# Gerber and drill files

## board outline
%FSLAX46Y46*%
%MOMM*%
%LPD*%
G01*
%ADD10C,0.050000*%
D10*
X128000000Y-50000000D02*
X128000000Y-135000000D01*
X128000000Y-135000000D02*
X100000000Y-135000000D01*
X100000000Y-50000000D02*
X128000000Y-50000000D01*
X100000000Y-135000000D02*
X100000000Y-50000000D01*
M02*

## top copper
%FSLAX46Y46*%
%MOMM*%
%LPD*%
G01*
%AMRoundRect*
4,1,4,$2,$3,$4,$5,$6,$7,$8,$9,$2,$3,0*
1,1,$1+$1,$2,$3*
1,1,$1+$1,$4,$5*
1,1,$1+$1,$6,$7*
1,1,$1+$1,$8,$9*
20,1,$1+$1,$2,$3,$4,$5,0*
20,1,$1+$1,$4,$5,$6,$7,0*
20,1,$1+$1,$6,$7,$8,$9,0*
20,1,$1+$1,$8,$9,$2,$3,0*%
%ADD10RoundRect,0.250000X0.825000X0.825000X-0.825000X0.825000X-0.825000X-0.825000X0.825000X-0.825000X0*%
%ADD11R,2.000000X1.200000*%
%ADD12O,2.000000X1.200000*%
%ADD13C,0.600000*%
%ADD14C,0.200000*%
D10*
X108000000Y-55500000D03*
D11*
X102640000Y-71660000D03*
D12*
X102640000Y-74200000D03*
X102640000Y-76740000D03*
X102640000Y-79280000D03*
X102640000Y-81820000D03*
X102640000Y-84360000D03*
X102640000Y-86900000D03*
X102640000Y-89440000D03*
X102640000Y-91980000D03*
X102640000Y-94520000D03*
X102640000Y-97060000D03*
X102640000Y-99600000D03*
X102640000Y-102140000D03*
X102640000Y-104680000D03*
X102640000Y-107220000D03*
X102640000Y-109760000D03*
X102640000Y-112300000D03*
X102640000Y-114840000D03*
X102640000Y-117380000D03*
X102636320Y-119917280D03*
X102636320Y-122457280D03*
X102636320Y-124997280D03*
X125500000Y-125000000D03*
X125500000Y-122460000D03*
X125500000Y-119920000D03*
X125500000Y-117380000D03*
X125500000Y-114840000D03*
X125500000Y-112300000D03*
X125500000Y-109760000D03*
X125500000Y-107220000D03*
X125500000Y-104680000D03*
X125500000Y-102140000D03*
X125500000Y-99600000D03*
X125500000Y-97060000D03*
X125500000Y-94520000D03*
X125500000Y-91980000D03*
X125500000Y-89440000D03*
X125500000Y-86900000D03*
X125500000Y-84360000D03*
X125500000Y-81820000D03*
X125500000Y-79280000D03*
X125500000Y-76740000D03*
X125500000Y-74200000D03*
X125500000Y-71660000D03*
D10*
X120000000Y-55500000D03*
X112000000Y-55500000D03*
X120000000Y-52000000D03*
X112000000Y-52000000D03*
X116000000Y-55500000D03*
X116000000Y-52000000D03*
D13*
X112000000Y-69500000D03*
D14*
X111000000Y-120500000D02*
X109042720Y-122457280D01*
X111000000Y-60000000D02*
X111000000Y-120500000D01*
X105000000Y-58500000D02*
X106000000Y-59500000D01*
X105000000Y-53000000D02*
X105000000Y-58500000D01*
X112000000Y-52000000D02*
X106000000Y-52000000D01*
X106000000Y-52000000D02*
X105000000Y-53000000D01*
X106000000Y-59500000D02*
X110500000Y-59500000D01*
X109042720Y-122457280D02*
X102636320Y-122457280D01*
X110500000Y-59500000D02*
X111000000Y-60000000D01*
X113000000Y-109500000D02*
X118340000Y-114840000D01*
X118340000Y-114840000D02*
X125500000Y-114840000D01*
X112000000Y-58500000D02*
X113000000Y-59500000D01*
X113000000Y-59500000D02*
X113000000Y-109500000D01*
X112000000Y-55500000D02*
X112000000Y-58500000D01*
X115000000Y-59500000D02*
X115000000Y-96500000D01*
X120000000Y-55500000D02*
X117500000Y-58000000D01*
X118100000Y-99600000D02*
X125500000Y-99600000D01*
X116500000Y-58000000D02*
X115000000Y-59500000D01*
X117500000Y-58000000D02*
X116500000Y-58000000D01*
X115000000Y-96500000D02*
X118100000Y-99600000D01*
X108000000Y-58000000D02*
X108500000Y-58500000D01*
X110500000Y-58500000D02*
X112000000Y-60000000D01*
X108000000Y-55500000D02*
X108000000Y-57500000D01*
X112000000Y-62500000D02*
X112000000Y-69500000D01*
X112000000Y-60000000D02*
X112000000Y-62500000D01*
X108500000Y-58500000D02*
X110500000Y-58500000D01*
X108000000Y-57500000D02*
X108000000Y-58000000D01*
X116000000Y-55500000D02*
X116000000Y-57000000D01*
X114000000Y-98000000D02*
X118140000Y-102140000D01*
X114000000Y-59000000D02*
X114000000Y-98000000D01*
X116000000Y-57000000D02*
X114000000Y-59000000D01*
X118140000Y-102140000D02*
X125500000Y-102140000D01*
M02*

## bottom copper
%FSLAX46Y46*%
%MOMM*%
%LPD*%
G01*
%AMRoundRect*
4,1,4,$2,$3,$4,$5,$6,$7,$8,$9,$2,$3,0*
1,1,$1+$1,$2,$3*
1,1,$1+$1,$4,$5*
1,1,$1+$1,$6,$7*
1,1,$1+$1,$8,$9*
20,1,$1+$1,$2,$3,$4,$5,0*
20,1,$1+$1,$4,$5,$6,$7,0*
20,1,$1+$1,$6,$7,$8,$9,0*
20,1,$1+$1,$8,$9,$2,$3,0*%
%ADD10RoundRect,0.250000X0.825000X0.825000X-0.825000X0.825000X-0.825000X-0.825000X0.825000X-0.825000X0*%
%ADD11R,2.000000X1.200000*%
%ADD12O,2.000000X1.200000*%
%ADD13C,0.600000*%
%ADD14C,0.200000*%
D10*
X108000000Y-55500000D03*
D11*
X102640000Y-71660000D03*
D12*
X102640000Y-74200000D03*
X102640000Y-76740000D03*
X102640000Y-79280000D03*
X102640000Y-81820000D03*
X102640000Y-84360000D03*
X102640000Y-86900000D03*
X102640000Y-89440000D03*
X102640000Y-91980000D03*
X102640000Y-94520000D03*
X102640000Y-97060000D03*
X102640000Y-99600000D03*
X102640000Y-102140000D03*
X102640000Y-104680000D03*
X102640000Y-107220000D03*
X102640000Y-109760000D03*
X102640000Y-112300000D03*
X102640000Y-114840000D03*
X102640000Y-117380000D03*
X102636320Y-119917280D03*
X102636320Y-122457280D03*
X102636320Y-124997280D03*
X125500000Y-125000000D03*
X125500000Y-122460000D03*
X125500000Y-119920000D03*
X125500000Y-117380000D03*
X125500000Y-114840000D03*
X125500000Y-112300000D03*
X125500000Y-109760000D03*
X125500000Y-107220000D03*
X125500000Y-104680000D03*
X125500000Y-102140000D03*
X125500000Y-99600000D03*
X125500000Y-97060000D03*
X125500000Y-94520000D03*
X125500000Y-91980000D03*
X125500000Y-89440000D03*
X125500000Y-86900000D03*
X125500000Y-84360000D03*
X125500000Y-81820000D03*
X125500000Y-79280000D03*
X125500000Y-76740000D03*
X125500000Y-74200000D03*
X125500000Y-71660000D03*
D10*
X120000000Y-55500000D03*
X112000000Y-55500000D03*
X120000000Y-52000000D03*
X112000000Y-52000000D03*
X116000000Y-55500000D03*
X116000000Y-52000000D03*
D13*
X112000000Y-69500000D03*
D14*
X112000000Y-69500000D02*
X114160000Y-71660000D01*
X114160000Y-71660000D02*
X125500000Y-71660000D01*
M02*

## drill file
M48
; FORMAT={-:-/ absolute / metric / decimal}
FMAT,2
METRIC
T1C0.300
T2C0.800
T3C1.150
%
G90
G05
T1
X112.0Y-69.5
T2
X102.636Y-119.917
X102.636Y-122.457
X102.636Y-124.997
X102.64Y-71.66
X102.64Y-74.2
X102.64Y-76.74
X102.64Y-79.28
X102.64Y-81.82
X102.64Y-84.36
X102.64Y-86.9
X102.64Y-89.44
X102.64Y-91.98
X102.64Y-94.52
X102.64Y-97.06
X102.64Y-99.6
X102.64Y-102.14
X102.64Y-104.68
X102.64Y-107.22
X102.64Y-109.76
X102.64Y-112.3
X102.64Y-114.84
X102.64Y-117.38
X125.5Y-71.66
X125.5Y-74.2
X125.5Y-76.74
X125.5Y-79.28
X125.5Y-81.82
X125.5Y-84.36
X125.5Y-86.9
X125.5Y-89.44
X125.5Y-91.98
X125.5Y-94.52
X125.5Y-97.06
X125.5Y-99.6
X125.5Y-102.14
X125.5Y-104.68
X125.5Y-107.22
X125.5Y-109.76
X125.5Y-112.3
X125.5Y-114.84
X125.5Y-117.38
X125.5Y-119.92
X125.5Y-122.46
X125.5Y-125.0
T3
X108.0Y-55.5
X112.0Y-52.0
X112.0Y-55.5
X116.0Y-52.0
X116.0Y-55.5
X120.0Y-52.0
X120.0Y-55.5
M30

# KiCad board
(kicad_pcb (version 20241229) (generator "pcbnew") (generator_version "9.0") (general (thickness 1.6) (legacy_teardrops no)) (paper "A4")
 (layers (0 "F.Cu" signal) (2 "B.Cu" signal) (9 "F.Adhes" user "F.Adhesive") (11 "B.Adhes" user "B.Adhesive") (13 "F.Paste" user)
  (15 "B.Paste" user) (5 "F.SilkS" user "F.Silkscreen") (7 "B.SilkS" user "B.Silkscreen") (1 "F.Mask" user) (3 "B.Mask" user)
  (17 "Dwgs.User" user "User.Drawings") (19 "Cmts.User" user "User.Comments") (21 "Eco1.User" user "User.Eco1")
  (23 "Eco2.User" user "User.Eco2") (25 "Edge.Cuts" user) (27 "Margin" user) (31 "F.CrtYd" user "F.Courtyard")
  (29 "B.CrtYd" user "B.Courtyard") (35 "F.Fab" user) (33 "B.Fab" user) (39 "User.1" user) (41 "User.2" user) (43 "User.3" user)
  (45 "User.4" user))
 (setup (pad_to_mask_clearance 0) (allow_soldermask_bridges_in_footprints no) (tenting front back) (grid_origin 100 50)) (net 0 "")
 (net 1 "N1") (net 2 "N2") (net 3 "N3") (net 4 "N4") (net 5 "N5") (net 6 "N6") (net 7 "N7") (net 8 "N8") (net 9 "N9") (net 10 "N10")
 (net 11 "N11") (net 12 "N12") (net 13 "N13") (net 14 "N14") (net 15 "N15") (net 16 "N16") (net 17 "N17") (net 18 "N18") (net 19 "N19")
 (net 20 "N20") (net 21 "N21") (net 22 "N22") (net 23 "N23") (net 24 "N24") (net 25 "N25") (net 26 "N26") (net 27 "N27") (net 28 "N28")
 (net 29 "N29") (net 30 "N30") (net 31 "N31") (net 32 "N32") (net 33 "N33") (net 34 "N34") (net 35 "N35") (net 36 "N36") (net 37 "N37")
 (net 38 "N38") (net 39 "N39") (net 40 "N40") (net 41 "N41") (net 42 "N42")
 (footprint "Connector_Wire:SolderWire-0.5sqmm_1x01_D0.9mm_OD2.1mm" (layer "F.Cu") (at 108 55.5 180)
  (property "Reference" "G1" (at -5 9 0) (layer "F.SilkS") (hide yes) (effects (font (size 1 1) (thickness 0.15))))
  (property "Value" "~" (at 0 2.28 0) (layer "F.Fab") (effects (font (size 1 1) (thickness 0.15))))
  (pad "1" thru_hole roundrect (at 0 0 180) (size 2.15 2.15) (drill 1.15) (layers "*.Cu" "*.Mask") (remove_unused_layers no)
   (roundrect_rratio 0.116279) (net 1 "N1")))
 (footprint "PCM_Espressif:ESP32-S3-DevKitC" (layer "F.Cu") (at 102.64 71.66)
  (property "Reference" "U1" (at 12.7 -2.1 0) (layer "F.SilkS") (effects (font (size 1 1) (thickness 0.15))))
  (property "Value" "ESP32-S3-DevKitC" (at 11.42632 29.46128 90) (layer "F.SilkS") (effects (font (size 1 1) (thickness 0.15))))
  (pad "1" thru_hole rect (at 0 0 270) (size 1.2 2) (drill 0.8) (layers "*.Cu" "*.Mask") (remove_unused_layers no) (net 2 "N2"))
  (pad "2" thru_hole oval (at 0 2.54 270) (size 1.2 2) (drill 0.8) (layers "*.Cu" "*.Mask") (remove_unused_layers no) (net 2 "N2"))
  (pad "3" thru_hole oval (at 0 5.08 270) (size 1.2 2) (drill 0.8) (layers "*.Cu" "*.Mask") (remove_unused_layers no) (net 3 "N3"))
  (pad "4" thru_hole oval (at 0 7.62 270) (size 1.2 2) (drill 0.8) (layers "*.Cu" "*.Mask") (remove_unused_layers no) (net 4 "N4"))
  (pad "5" thru_hole oval (at 0 10.16 270) (size 1.2 2) (drill 0.8) (layers "*.Cu" "*.Mask") (remove_unused_layers no) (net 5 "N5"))
  (pad "6" thru_hole oval (at 0 12.7 270) (size 1.2 2) (drill 0.8) (layers "*.Cu" "*.Mask") (remove_unused_layers no) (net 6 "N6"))
  (pad "7" thru_hole oval (at 0 15.24 270) (size 1.2 2) (drill 0.8) (layers "*.Cu" "*.Mask") (remove_unused_layers no) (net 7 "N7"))
  (pad "8" thru_hole oval (at 0 17.78 270) (size 1.2 2) (drill 0.8) (layers "*.Cu" "*.Mask") (remove_unused_layers no) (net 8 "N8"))
  (pad "9" thru_hole oval (at 0 20.32 270) (size 1.2 2) (drill 0.8) (layers "*.Cu" "*.Mask") (remove_unused_layers no) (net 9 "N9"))
  (pad "10" thru_hole oval (at 0 22.86 270) (size 1.2 2) (drill 0.8) (layers "*.Cu" "*.Mask") (remove_unused_layers no) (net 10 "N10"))
  (pad "11" thru_hole oval (at 0 25.4 270) (size 1.2 2) (drill 0.8) (layers "*.Cu" "*.Mask") (remove_unused_layers no) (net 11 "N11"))
  (pad "12" thru_hole oval (at 0 27.94 270) (size 1.2 2) (drill 0.8) (layers "*.Cu" "*.Mask") (remove_unused_layers no) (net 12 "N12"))
  (pad "13" thru_hole oval (at 0 30.48 270) (size 1.2 2) (drill 0.8) (layers "*.Cu" "*.Mask") (remove_unused_layers no) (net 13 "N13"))
  (pad "14" thru_hole oval (at 0 33.02 270) (size 1.2 2) (drill 0.8) (layers "*.Cu" "*.Mask") (remove_unused_layers no) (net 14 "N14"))
  (pad "15" thru_hole oval (at 0 35.56 270) (size 1.2 2) (drill 0.8) (layers "*.Cu" "*.Mask") (remove_unused_layers no) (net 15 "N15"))
  (pad "16" thru_hole oval (at 0 38.1 270) (size 1.2 2) (drill 0.8) (layers "*.Cu" "*.Mask") (remove_unused_layers no) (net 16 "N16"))
  (pad "17" thru_hole oval (at 0 40.64 270) (size 1.2 2) (drill 0.8) (layers "*.Cu" "*.Mask") (remove_unused_layers no) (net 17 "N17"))
  (pad "18" thru_hole oval (at 0 43.18 270) (size 1.2 2) (drill 0.8) (layers "*.Cu" "*.Mask") (remove_unused_layers no) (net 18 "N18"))
  (pad "19" thru_hole oval (at 0 45.72 270) (size 1.2 2) (drill 0.8) (layers "*.Cu" "*.Mask") (remove_unused_layers no) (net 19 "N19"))
  (pad "20" thru_hole oval (at -0.00368 48.25728 270) (size 1.2 2) (drill 0.8) (layers "*.Cu" "*.Mask") (remove_unused_layers no)
   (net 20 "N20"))
  (pad "21" thru_hole oval (at -0.00368 50.79728 270) (size 1.2 2) (drill 0.8) (layers "*.Cu" "*.Mask") (remove_unused_layers no)
   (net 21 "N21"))
  (pad "22" thru_hole oval (at -0.00368 53.33728 270) (size 1.2 2) (drill 0.8) (layers "*.Cu" "*.Mask") (remove_unused_layers no)
   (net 1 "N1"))
  (pad "23" thru_hole oval (at 22.86 53.34 270) (size 1.2 2) (drill 0.8) (layers "*.Cu" "*.Mask") (remove_unused_layers no) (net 1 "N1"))
  (pad "24" thru_hole oval (at 22.86 50.8 270) (size 1.2 2) (drill 0.8) (layers "*.Cu" "*.Mask") (remove_unused_layers no) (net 1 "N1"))
  (pad "25" thru_hole oval (at 22.86 48.26 270) (size 1.2 2) (drill 0.8) (layers "*.Cu" "*.Mask") (remove_unused_layers no) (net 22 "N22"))
  (pad "26" thru_hole oval (at 22.86 45.72 270) (size 1.2 2) (drill 0.8) (layers "*.Cu" "*.Mask") (remove_unused_layers no) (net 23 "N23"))
  (pad "27" thru_hole oval (at 22.86 43.18 270) (size 1.2 2) (drill 0.8) (layers "*.Cu" "*.Mask") (remove_unused_layers no) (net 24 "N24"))
  (pad "28" thru_hole oval (at 22.86 40.64 270) (size 1.2 2) (drill 0.8) (layers "*.Cu" "*.Mask") (remove_unused_layers no) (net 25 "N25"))
  (pad "29" thru_hole oval (at 22.86 38.1 270) (size 1.2 2) (drill 0.8) (layers "*.Cu" "*.Mask") (remove_unused_layers no) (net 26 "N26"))
  (pad "30" thru_hole oval (at 22.86 35.56 270) (size 1.2 2) (drill 0.8) (layers "*.Cu" "*.Mask") (remove_unused_layers no) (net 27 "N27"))
  (pad "31" thru_hole oval (at 22.86 33.02 270) (size 1.2 2) (drill 0.8) (layers "*.Cu" "*.Mask") (remove_unused_layers no) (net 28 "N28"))
  (pad "32" thru_hole oval (at 22.86 30.48 270) (size 1.2 2) (drill 0.8) (layers "*.Cu" "*.Mask") (remove_unused_layers no) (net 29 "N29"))
  (pad "33" thru_hole oval (at 22.86 27.94 270) (size 1.2 2) (drill 0.8) (layers "*.Cu" "*.Mask") (remove_unused_layers no) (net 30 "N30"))
  (pad "34" thru_hole oval (at 22.86 25.4 270) (size 1.2 2) (drill 0.8) (layers "*.Cu" "*.Mask") (remove_unused_layers no) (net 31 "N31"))
  (pad "35" thru_hole oval (at 22.86 22.86 270) (size 1.2 2) (drill 0.8) (layers "*.Cu" "*.Mask") (remove_unused_layers no) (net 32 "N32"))
  (pad "36" thru_hole oval (at 22.86 20.32 270) (size 1.2 2) (drill 0.8) (layers "*.Cu" "*.Mask") (remove_unused_layers no) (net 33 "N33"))
  (pad "37" thru_hole oval (at 22.86 17.78 270) (size 1.2 2) (drill 0.8) (layers "*.Cu" "*.Mask") (remove_unused_layers no) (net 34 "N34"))
  (pad "38" thru_hole oval (at 22.86 15.24 270) (size 1.2 2) (drill 0.8) (layers "*.Cu" "*.Mask") (remove_unused_layers no) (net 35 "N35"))
  (pad "39" thru_hole oval (at 22.86 12.7 270) (size 1.2 2) (drill 0.8) (layers "*.Cu" "*.Mask") (remove_unused_layers no) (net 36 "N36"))
  (pad "40" thru_hole oval (at 22.86 10.16 270) (size 1.2 2) (drill 0.8) (layers "*.Cu" "*.Mask") (remove_unused_layers no) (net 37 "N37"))
  (pad "41" thru_hole oval (at 22.86 7.62 270) (size 1.2 2) (drill 0.8) (layers "*.Cu" "*.Mask") (remove_unused_layers no) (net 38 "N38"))
  (pad "42" thru_hole oval (at 22.86 5.08 270) (size 1.2 2) (drill 0.8) (layers "*.Cu" "*.Mask") (remove_unused_layers no) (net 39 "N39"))
  (pad "43" thru_hole oval (at 22.86 2.54 270) (size 1.2 2) (drill 0.8) (layers "*.Cu" "*.Mask") (remove_unused_layers no) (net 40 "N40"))
  (pad "44" thru_hole oval (at 22.86 0 270) (size 1.2 2) (drill 0.8) (layers "*.Cu" "*.Mask") (remove_unused_layers no) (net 1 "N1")))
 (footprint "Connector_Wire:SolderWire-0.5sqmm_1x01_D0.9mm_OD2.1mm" (layer "F.Cu") (at 120 55.5 180)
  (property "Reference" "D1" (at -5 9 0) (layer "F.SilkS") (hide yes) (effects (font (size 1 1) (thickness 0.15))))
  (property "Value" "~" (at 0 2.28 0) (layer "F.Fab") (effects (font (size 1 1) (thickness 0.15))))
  (pad "1" thru_hole roundrect (at 0 0 180) (size 2.15 2.15) (drill 1.15) (layers "*.Cu" "*.Mask") (remove_unused_layers no)
   (roundrect_rratio 0.116279) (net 30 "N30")))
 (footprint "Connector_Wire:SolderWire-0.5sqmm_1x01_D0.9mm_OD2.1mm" (layer "F.Cu") (at 112 55.5 180)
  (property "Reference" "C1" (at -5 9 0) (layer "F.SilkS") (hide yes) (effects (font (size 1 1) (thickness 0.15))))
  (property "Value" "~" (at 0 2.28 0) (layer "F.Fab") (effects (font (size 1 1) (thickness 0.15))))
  (pad "1" thru_hole roundrect (at 0 0 180) (size 2.15 2.15) (drill 1.15) (layers "*.Cu" "*.Mask") (remove_unused_layers no)
   (roundrect_rratio 0.116279) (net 24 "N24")))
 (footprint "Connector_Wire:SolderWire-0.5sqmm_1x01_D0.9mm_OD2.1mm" (layer "F.Cu") (at 120 52 180)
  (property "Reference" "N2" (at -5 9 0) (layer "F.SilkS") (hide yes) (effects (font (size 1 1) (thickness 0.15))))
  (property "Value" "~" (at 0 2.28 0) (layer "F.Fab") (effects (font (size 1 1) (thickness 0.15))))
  (pad "1" thru_hole roundrect (at 0 0 180) (size 2.15 2.15) (drill 1.15) (layers "*.Cu" "*.Mask") (remove_unused_layers no)
   (roundrect_rratio 0.116279) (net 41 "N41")))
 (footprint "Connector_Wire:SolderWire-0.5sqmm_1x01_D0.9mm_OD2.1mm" (layer "F.Cu") (at 112 52 180)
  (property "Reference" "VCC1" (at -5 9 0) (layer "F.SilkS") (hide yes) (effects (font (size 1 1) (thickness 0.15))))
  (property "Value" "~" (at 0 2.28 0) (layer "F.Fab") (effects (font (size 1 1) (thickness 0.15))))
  (pad "1" thru_hole roundrect (at 0 0 180) (size 2.15 2.15) (drill 1.15) (layers "*.Cu" "*.Mask") (remove_unused_layers no)
   (roundrect_rratio 0.116279) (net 21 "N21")))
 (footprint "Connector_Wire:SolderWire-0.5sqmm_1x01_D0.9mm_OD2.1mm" (layer "F.Cu") (at 116 55.5 180)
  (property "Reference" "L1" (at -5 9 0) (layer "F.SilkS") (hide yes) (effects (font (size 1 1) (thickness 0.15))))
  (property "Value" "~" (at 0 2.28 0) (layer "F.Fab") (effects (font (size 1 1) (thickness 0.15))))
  (pad "1" thru_hole roundrect (at 0 0 180) (size 2.15 2.15) (drill 1.15) (layers "*.Cu" "*.Mask") (remove_unused_layers no)
   (roundrect_rratio 0.116279) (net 29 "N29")))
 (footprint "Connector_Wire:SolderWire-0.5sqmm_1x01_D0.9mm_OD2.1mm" (layer "F.Cu") (at 116 52 180)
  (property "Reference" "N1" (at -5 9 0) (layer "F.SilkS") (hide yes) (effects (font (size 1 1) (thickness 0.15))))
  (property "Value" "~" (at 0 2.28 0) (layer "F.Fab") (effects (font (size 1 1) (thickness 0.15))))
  (pad "1" thru_hole roundrect (at 0 0 180) (size 2.15 2.15) (drill 1.15) (layers "*.Cu" "*.Mask") (remove_unused_layers no)
   (roundrect_rratio 0.116279) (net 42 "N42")))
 (gr_line (start 128 50) (end 128 135) (stroke (width 0.05) (type default)) (layer "Edge.Cuts"))
 (gr_line (start 128 135) (end 100 135) (stroke (width 0.05) (type default)) (layer "Edge.Cuts"))
 (gr_line (start 100 50) (end 128 50) (stroke (width 0.05) (type default)) (layer "Edge.Cuts"))
 (gr_line (start 100 135) (end 100 50) (stroke (width 0.05) (type default)) (layer "Edge.Cuts"))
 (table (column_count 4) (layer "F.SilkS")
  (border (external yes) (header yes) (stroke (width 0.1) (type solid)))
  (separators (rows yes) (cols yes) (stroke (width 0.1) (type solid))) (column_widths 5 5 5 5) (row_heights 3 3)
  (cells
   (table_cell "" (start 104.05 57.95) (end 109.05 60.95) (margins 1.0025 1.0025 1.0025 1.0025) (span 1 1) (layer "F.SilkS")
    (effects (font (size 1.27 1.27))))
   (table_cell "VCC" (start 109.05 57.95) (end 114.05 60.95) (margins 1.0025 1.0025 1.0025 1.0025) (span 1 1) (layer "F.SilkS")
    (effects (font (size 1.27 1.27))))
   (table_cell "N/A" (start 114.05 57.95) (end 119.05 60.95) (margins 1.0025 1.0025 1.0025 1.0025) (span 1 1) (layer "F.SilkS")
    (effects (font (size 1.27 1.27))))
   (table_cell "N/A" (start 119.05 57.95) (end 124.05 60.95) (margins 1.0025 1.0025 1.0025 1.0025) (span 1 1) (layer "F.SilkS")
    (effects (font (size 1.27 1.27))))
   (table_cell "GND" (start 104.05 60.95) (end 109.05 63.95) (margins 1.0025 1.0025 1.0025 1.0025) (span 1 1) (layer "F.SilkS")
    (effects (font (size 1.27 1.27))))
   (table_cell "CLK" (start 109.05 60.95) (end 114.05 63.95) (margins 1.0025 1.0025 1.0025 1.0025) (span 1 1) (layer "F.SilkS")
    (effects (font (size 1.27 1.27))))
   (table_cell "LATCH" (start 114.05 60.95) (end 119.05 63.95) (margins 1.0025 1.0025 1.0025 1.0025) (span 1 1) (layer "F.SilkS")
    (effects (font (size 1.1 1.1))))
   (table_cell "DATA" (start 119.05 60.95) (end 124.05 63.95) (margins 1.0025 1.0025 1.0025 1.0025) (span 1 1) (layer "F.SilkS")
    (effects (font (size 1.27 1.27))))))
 (segment (start 111 120.5) (end 109.04272 122.45728) (width 0.2) (layer "F.Cu") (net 21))
 (segment (start 111 60) (end 111 120.5) (width 0.2) (layer "F.Cu") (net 21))
 (segment (start 105 58.5) (end 106 59.5) (width 0.2) (layer "F.Cu") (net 21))
 (segment (start 105 53) (end 105 58.5) (width 0.2) (layer "F.Cu") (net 21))
 (segment (start 112 52) (end 106 52) (width 0.2) (layer "F.Cu") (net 21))
 (segment (start 106 52) (end 105 53) (width 0.2) (layer "F.Cu") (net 21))
 (segment (start 106 59.5) (end 110.5 59.5) (width 0.2) (layer "F.Cu") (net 21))
 (segment (start 109.04272 122.45728) (end 102.63632 122.45728) (width 0.2) (layer "F.Cu") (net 21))
 (segment (start 110.5 59.5) (end 111 60) (width 0.2) (layer "F.Cu") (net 21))
 (segment (start 113 109.5) (end 118.34 114.84) (width 0.2) (layer "F.Cu") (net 24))
 (segment (start 118.34 114.84) (end 125.5 114.84) (width 0.2) (layer "F.Cu") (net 24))
 (segment (start 112 58.5) (end 113 59.5) (width 0.2) (layer "F.Cu") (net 24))
 (segment (start 113 59.5) (end 113 109.5) (width 0.2) (layer "F.Cu") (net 24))
 (segment (start 112 55.5) (end 112 58.5) (width 0.2) (layer "F.Cu") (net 24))
 (segment (start 115 59.5) (end 115 96.5) (width 0.2) (layer "F.Cu") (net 30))
 (segment (start 120 55.5) (end 117.5 58) (width 0.2) (layer "F.Cu") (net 30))
 (segment (start 118.1 99.6) (end 125.5 99.6) (width 0.2) (layer "F.Cu") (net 30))
 (segment (start 116.5 58) (end 115 59.5) (width 0.2) (layer "F.Cu") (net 30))
 (segment (start 117.5 58) (end 116.5 58) (width 0.2) (layer "F.Cu") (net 30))
 (segment (start 115 96.5) (end 118.1 99.6) (width 0.2) (layer "F.Cu") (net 30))
 (segment (start 108 58) (end 108.5 58.5) (width 0.2) (layer "F.Cu") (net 1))
 (segment (start 110.5 58.5) (end 112 60) (width 0.2) (layer "F.Cu") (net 1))
 (segment (start 108 55.5) (end 108 57.5) (width 0.2) (layer "F.Cu") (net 1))
 (segment (start 112 62.5) (end 112 69.5) (width 0.2) (layer "F.Cu") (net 1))
 (segment (start 112 60) (end 112 62.5) (width 0.2) (layer "F.Cu") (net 1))
 (segment (start 108.5 58.5) (end 110.5 58.5) (width 0.2) (layer "F.Cu") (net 1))
 (segment (start 108 57.5) (end 108 58) (width 0.2) (layer "F.Cu") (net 1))
 (via (at 112 69.5) (size 0.6) (drill 0.3) (layers "F.Cu" "B.Cu") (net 1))
 (segment (start 112 69.5) (end 114.16 71.66) (width 0.2) (layer "B.Cu") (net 1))
 (segment (start 114.16 71.66) (end 125.5 71.66) (width 0.2) (layer "B.Cu") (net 1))
 (segment (start 116 55.5) (end 116 57) (width 0.2) (layer "F.Cu") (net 29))
 (segment (start 114 98) (end 118.14 102.14) (width 0.2) (layer "F.Cu") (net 29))
 (segment (start 114 59) (end 114 98) (width 0.2) (layer "F.Cu") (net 29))
 (segment (start 116 57) (end 114 59) (width 0.2) (layer "F.Cu") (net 29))
 (segment (start 118.14 102.14) (end 125.5 102.14) (width 0.2) (layer "F.Cu") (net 29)))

